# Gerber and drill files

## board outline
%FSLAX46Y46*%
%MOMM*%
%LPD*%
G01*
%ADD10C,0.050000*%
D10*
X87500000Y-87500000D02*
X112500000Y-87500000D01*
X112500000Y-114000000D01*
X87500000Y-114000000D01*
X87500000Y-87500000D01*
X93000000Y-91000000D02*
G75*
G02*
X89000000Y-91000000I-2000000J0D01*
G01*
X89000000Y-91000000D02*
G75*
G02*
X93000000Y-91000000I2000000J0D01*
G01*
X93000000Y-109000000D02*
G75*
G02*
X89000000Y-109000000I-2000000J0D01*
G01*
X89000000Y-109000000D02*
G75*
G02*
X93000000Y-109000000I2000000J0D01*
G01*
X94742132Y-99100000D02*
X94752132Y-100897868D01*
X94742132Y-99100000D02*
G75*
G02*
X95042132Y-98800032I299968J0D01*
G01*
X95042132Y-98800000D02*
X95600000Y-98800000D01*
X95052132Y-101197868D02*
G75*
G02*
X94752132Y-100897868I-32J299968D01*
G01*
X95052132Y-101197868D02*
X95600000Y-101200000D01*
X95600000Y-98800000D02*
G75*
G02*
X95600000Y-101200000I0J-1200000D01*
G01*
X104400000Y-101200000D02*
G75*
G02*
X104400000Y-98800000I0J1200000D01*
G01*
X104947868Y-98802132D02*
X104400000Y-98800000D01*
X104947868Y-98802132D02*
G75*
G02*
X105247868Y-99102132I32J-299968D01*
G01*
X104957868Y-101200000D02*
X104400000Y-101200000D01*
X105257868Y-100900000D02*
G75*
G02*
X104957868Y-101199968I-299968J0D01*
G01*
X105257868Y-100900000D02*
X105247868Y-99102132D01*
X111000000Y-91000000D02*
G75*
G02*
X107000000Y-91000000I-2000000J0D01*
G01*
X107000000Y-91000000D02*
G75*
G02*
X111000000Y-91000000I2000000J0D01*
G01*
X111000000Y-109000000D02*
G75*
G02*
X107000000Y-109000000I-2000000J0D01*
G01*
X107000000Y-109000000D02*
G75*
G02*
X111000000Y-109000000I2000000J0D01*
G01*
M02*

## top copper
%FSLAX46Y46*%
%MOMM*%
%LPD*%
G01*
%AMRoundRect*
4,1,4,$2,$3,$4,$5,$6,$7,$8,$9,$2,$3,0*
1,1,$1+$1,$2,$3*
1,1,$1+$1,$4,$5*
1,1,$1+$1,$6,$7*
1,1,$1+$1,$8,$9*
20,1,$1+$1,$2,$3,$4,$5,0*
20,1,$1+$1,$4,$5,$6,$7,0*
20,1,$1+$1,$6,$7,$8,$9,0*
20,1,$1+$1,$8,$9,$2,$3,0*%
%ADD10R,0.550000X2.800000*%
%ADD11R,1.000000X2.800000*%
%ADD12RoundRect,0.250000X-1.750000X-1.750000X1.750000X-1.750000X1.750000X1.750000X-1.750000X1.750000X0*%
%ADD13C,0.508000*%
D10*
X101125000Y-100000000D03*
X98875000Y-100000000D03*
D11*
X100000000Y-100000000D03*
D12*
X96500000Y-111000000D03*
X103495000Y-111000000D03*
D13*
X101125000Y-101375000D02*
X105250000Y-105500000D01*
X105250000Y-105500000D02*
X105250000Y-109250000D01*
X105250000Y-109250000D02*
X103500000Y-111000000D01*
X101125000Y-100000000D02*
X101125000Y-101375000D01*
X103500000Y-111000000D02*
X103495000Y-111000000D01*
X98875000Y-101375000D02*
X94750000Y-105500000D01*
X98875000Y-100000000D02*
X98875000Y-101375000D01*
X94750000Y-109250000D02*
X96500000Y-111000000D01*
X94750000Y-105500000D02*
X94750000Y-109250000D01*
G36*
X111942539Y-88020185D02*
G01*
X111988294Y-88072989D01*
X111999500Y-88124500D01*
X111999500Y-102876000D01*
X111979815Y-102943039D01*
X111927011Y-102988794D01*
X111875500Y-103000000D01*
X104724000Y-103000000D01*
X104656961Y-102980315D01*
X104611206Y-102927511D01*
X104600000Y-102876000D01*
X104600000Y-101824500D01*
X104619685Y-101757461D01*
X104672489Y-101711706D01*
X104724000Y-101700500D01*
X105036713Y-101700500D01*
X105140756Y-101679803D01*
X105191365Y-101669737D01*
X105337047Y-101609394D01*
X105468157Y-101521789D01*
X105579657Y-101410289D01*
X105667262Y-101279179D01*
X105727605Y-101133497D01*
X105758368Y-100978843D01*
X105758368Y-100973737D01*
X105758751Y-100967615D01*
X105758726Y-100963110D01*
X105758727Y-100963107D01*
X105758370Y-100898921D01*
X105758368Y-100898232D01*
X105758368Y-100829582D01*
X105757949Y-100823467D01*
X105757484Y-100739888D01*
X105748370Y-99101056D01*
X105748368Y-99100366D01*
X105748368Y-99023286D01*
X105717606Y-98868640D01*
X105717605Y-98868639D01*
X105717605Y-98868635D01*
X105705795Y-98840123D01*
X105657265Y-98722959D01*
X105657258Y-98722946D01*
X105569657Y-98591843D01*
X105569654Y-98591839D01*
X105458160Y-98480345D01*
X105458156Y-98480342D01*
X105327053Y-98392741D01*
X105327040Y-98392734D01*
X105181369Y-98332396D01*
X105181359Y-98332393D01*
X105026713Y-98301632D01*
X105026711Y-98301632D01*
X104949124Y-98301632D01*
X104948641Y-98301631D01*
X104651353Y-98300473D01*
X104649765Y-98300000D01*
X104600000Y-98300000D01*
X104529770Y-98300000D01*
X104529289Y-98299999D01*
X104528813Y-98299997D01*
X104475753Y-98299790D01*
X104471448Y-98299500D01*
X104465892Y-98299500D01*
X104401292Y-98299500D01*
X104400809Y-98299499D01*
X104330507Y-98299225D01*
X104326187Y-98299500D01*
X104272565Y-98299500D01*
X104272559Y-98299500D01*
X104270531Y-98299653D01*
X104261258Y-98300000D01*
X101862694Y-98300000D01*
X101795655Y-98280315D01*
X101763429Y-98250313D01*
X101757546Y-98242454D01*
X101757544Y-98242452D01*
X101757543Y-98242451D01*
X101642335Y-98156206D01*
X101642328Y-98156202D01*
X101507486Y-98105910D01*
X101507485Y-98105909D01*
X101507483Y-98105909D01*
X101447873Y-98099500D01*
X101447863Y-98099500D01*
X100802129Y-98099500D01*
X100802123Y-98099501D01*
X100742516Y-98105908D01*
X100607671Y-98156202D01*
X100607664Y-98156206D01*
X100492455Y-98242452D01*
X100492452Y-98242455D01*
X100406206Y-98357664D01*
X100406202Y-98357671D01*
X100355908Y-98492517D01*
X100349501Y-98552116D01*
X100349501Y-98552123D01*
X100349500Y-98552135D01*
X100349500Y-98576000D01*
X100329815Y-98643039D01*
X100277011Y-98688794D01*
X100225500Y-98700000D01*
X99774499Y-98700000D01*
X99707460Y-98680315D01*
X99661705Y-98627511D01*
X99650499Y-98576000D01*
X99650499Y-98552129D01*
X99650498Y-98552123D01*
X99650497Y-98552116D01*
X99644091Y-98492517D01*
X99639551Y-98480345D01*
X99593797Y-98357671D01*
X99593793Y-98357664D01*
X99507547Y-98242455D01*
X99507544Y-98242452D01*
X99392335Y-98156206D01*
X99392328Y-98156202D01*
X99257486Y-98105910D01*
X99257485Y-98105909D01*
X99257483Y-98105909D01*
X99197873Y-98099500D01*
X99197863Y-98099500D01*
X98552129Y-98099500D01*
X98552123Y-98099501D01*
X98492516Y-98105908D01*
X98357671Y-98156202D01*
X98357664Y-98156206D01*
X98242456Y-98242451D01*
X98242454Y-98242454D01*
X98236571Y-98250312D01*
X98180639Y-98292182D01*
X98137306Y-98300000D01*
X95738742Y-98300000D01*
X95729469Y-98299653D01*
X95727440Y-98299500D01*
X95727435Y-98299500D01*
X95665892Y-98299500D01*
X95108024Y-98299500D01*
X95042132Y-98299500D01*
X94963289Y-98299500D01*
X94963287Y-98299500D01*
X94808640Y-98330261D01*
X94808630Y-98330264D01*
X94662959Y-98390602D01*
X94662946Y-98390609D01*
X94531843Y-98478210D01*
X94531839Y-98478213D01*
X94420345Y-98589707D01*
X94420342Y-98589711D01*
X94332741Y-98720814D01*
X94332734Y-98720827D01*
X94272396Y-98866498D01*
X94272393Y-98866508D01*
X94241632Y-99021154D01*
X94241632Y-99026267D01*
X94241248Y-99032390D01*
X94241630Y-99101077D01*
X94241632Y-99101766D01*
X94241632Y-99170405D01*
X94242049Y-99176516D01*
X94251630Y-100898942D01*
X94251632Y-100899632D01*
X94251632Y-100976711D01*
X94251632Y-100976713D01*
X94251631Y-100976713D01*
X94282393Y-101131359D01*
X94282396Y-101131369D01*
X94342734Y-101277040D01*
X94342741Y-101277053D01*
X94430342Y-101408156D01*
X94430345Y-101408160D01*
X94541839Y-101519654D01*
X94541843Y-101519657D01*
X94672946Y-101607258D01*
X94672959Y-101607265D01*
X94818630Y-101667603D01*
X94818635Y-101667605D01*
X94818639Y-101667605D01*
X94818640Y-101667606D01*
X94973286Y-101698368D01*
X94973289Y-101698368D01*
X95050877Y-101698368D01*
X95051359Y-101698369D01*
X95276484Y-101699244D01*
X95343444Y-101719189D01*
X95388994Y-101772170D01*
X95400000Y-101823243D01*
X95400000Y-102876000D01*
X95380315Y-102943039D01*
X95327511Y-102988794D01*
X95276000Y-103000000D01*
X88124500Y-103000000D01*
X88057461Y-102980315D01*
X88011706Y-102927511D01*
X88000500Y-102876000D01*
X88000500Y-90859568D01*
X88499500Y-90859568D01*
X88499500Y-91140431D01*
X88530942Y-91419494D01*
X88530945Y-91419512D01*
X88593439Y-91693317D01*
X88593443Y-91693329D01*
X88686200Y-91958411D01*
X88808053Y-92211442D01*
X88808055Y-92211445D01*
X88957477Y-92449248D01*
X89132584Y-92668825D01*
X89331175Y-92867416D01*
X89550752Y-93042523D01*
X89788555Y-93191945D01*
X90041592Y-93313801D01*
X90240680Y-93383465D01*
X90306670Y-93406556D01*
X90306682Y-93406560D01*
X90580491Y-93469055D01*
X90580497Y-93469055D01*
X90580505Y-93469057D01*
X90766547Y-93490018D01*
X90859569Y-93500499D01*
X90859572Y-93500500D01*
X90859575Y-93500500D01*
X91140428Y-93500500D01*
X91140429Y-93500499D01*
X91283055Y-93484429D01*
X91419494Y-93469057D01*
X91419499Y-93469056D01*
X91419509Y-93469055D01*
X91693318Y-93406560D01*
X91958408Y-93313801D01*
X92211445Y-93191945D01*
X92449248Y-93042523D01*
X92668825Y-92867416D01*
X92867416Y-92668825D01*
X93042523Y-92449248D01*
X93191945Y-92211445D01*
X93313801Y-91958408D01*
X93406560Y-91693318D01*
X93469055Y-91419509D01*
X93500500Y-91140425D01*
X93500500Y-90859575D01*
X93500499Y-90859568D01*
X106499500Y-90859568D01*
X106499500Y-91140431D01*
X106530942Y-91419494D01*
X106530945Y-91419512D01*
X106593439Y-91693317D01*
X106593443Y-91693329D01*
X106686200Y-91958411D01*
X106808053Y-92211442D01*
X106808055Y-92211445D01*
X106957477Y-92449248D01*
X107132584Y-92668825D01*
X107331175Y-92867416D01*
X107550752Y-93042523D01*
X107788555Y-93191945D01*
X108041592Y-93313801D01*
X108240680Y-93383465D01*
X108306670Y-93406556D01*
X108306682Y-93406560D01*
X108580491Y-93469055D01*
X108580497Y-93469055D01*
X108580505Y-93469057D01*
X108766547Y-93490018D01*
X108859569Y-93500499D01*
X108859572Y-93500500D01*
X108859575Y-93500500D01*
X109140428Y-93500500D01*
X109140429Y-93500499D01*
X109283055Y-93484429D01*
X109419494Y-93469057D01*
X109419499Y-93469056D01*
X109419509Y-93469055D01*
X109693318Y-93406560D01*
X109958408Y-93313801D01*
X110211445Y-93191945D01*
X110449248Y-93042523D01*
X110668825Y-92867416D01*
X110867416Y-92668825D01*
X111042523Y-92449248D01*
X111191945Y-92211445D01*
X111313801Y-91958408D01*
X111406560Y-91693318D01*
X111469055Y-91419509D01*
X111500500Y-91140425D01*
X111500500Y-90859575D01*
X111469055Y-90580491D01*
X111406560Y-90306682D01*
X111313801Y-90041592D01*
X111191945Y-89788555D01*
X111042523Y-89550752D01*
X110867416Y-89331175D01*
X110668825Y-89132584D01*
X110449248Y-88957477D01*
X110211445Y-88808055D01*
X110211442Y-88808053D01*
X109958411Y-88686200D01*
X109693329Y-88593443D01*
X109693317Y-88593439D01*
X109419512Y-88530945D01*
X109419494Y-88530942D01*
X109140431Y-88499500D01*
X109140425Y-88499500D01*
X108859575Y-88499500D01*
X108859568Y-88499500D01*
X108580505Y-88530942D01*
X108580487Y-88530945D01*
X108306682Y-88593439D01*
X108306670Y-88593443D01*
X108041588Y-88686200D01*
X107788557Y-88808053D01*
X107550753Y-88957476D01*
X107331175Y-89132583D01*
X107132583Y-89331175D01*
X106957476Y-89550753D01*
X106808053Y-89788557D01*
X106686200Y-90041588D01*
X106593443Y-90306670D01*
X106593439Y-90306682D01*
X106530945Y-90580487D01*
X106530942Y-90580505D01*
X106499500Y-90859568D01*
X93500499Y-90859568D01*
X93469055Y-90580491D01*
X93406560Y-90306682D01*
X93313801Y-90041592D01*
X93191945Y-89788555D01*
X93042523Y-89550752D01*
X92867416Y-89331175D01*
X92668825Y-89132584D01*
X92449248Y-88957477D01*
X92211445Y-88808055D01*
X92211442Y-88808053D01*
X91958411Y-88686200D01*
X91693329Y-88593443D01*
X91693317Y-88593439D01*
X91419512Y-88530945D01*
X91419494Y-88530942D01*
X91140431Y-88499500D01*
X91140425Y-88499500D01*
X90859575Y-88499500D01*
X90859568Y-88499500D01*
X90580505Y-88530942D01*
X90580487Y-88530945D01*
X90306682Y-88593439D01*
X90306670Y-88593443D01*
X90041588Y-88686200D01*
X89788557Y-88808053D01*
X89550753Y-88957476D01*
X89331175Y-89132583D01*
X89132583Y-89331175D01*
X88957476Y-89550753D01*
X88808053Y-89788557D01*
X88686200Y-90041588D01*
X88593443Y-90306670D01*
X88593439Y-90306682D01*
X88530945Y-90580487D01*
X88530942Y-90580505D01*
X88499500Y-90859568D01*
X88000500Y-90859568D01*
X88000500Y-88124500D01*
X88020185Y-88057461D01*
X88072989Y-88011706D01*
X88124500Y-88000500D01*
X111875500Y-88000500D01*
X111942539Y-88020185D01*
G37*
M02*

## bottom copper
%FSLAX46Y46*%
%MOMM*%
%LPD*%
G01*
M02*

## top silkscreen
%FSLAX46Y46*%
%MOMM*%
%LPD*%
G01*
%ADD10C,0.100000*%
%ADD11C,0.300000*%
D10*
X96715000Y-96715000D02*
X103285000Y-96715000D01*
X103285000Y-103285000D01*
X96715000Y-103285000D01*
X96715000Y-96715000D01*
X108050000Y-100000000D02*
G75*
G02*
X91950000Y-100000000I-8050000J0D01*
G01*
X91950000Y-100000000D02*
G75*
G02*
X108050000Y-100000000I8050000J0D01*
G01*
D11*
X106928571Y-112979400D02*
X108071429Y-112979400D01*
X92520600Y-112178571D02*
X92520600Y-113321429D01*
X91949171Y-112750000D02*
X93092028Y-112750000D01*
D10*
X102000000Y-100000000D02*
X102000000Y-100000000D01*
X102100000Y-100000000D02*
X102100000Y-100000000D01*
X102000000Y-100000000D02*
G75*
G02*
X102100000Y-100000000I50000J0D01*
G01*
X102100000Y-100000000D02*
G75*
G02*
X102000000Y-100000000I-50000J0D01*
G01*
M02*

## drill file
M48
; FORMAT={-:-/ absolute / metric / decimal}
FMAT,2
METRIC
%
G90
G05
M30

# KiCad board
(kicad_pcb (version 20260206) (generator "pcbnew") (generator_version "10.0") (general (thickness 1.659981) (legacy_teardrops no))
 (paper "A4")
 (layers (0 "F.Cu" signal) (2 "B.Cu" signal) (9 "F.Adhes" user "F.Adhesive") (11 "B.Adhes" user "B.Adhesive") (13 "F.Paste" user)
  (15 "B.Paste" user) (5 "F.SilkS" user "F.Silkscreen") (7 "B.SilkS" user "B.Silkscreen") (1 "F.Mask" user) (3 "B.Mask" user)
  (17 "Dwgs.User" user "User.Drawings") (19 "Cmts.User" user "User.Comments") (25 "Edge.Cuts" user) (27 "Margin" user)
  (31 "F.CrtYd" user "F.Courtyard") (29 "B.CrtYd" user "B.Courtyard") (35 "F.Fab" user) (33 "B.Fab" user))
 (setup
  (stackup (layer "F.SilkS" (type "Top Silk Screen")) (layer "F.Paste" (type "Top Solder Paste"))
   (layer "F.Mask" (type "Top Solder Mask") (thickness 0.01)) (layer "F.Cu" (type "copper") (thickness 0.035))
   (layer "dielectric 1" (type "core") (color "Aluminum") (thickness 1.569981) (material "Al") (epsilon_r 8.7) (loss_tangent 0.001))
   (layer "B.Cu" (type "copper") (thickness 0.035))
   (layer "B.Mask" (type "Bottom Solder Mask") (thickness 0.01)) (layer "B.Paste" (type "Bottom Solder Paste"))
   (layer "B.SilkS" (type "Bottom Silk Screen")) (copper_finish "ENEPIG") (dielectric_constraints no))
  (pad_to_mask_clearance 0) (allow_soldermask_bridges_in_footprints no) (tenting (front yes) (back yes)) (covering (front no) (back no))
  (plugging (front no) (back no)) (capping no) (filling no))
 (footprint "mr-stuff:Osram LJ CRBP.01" (layer "F.Cu") (at 100 100 -90)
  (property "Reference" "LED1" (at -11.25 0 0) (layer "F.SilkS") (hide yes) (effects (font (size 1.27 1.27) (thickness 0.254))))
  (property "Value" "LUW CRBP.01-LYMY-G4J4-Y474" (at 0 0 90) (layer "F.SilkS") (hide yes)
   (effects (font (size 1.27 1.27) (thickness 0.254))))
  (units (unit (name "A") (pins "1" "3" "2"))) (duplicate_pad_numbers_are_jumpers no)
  (fp_line (start 0 -2) (end 0 -2) (stroke (width 0.1) (type solid)) (layer "F.SilkS"))
  (fp_line (start 0 -2.1) (end 0 -2.1) (stroke (width 0.1) (type solid)) (layer "F.SilkS"))
  (fp_arc (start 0 -2) (mid -0.05 -2.05) (end 0 -2.1) (stroke (width 0.1) (type solid)) (layer "F.SilkS"))
  (fp_arc (start 0 -2.1) (mid 0.05 -2.05) (end 0 -2) (stroke (width 0.1) (type solid)) (layer "F.SilkS"))
  (pad "1" smd rect (at 0 -1.125) (size 0.55 2.8) (layers "F.Cu" "F.Mask" "F.Paste") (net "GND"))
  (pad "2" smd rect (at 0 1.125) (size 0.55 2.8) (layers "F.Cu" "F.Mask" "F.Paste") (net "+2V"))
  (pad "3" smd rect (at 0 0) (size 1 2.8) (layers "F.Cu" "F.Mask" "F.Paste") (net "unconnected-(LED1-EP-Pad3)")))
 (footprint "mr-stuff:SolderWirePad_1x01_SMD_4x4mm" (layer "F.Cu") (at 96.5 111)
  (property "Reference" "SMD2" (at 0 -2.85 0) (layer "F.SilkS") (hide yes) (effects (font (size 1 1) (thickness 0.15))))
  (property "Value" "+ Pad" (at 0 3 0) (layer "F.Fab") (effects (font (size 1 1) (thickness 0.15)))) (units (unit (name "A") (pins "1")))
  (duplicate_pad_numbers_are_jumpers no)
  (pad "1" smd roundrect (at 0 0) (size 4 4) (layers "F.Cu" "F.Mask") (roundrect_rratio 0.0625) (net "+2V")))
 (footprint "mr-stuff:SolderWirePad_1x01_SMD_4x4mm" (layer "F.Cu") (at 103.495 111)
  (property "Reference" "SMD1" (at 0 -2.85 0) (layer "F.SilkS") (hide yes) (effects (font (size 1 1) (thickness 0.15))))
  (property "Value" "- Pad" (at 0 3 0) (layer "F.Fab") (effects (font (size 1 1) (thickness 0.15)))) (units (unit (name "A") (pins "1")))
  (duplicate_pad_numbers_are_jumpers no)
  (pad "1" smd roundrect (at 0 0) (size 4 4) (layers "F.Cu" "F.Mask") (roundrect_rratio 0.0625) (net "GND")))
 (gr_rect (start 96.715 96.715) (end 103.285 103.285) (stroke (width 0.1) (type default)) (fill no) (layer "F.SilkS"))
 (gr_circle (center 100 100) (end 108.05 100) (stroke (width 0.1) (type default)) (fill no) (layer "F.SilkS"))
 (gr_rect (start 87.5 87.5) (end 112.5 114) (stroke (width 0.05) (type solid)) (fill no) (layer "Edge.Cuts"))
 (gr_circle (center 91 91) (end 91 93) (stroke (width 0.05) (type solid)) (fill no) (layer "Edge.Cuts"))
 (gr_circle (center 91 109) (end 91 111) (stroke (width 0.05) (type solid)) (fill no) (layer "Edge.Cuts"))
 (gr_line (start 94.742132 99.1) (end 94.752132 100.897868) (stroke (width 0.05) (type default)) (layer "Edge.Cuts"))
 (gr_arc (start 94.742132 99.1) (mid 94.83 98.887868) (end 95.042132 98.8) (stroke (width 0.05) (type default)) (layer "Edge.Cuts"))
 (gr_line (start 95.042132 98.8) (end 95.6 98.8) (stroke (width 0.05) (type default)) (layer "Edge.Cuts"))
 (gr_arc (start 95.052132 101.197868) (mid 94.84 101.11) (end 94.752132 100.897868) (stroke (width 0.05) (type default)) (layer "Edge.Cuts"))
 (gr_line (start 95.052132 101.197868) (end 95.6 101.2) (stroke (width 0.05) (type default)) (layer "Edge.Cuts"))
 (gr_arc (start 95.6 98.8) (mid 96.8 100) (end 95.6 101.2) (stroke (width 0.05) (type solid)) (layer "Edge.Cuts"))
 (gr_arc (start 104.4 101.2) (mid 103.2 100) (end 104.4 98.8) (stroke (width 0.05) (type solid)) (layer "Edge.Cuts"))
 (gr_line (start 104.947868 98.802132) (end 104.4 98.8) (stroke (width 0.05) (type default)) (layer "Edge.Cuts"))
 (gr_arc (start 104.947868 98.802132) (mid 105.16 98.89) (end 105.247868 99.102132) (stroke (width 0.05) (type default)) (layer "Edge.Cuts"))
 (gr_line (start 104.957868 101.2) (end 104.4 101.2) (stroke (width 0.05) (type default)) (layer "Edge.Cuts"))
 (gr_arc (start 105.257868 100.9) (mid 105.17 101.112132) (end 104.957868 101.2) (stroke (width 0.05) (type default)) (layer "Edge.Cuts"))
 (gr_line (start 105.257868 100.9) (end 105.247868 99.102132) (stroke (width 0.05) (type default)) (layer "Edge.Cuts"))
 (gr_circle (center 109 91) (end 109 93) (stroke (width 0.05) (type solid)) (fill no) (layer "Edge.Cuts"))
 (gr_circle (center 109 109) (end 109 111) (stroke (width 0.05) (type solid)) (fill no) (layer "Edge.Cuts"))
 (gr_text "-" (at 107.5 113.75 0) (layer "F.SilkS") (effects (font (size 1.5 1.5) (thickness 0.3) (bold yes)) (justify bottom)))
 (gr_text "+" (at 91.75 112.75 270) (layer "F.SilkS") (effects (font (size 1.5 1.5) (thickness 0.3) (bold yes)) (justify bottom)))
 (segment (start 101.125 101.375) (end 105.25 105.5) (width 0.508) (layer "F.Cu") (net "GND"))
 (segment (start 105.25 105.5) (end 105.25 109.25) (width 0.508) (layer "F.Cu") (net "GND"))
 (segment (start 105.25 109.25) (end 103.5 111) (width 0.508) (layer "F.Cu") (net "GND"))
 (segment (start 101.125 100) (end 101.125 101.375) (width 0.508) (layer "F.Cu") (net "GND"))
 (segment (start 103.5 111) (end 103.495 111) (width 0.508) (layer "F.Cu") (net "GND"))
 (segment (start 98.875 101.375) (end 94.75 105.5) (width 0.508) (layer "F.Cu") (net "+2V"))
 (segment (start 98.875 100) (end 98.875 101.375) (width 0.508) (layer "F.Cu") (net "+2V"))
 (segment (start 94.75 109.25) (end 96.5 111) (width 0.508) (layer "F.Cu") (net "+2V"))
 (segment (start 94.75 105.5) (end 94.75 109.25) (width 0.508) (layer "F.Cu") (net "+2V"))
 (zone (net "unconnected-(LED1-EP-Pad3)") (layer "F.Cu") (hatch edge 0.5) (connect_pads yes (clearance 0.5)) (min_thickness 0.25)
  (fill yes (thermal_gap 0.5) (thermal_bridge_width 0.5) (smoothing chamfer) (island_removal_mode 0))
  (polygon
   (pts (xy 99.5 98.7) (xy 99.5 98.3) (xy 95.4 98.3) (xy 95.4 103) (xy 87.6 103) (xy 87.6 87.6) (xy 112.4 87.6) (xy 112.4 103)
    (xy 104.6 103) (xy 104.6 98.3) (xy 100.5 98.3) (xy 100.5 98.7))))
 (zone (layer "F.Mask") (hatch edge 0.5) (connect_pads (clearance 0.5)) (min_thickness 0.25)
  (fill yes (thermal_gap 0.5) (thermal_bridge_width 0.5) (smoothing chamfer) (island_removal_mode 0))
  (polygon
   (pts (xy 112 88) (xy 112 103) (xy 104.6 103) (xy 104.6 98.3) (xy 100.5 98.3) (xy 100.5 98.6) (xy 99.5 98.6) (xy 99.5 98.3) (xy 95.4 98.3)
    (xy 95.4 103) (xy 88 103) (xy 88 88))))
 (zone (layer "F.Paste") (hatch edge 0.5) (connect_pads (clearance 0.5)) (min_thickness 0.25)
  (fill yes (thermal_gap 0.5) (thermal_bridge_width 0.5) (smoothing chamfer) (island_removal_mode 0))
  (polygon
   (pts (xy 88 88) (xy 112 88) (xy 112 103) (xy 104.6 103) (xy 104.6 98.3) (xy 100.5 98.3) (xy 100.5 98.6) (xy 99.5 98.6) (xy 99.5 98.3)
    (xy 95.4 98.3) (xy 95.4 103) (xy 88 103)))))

